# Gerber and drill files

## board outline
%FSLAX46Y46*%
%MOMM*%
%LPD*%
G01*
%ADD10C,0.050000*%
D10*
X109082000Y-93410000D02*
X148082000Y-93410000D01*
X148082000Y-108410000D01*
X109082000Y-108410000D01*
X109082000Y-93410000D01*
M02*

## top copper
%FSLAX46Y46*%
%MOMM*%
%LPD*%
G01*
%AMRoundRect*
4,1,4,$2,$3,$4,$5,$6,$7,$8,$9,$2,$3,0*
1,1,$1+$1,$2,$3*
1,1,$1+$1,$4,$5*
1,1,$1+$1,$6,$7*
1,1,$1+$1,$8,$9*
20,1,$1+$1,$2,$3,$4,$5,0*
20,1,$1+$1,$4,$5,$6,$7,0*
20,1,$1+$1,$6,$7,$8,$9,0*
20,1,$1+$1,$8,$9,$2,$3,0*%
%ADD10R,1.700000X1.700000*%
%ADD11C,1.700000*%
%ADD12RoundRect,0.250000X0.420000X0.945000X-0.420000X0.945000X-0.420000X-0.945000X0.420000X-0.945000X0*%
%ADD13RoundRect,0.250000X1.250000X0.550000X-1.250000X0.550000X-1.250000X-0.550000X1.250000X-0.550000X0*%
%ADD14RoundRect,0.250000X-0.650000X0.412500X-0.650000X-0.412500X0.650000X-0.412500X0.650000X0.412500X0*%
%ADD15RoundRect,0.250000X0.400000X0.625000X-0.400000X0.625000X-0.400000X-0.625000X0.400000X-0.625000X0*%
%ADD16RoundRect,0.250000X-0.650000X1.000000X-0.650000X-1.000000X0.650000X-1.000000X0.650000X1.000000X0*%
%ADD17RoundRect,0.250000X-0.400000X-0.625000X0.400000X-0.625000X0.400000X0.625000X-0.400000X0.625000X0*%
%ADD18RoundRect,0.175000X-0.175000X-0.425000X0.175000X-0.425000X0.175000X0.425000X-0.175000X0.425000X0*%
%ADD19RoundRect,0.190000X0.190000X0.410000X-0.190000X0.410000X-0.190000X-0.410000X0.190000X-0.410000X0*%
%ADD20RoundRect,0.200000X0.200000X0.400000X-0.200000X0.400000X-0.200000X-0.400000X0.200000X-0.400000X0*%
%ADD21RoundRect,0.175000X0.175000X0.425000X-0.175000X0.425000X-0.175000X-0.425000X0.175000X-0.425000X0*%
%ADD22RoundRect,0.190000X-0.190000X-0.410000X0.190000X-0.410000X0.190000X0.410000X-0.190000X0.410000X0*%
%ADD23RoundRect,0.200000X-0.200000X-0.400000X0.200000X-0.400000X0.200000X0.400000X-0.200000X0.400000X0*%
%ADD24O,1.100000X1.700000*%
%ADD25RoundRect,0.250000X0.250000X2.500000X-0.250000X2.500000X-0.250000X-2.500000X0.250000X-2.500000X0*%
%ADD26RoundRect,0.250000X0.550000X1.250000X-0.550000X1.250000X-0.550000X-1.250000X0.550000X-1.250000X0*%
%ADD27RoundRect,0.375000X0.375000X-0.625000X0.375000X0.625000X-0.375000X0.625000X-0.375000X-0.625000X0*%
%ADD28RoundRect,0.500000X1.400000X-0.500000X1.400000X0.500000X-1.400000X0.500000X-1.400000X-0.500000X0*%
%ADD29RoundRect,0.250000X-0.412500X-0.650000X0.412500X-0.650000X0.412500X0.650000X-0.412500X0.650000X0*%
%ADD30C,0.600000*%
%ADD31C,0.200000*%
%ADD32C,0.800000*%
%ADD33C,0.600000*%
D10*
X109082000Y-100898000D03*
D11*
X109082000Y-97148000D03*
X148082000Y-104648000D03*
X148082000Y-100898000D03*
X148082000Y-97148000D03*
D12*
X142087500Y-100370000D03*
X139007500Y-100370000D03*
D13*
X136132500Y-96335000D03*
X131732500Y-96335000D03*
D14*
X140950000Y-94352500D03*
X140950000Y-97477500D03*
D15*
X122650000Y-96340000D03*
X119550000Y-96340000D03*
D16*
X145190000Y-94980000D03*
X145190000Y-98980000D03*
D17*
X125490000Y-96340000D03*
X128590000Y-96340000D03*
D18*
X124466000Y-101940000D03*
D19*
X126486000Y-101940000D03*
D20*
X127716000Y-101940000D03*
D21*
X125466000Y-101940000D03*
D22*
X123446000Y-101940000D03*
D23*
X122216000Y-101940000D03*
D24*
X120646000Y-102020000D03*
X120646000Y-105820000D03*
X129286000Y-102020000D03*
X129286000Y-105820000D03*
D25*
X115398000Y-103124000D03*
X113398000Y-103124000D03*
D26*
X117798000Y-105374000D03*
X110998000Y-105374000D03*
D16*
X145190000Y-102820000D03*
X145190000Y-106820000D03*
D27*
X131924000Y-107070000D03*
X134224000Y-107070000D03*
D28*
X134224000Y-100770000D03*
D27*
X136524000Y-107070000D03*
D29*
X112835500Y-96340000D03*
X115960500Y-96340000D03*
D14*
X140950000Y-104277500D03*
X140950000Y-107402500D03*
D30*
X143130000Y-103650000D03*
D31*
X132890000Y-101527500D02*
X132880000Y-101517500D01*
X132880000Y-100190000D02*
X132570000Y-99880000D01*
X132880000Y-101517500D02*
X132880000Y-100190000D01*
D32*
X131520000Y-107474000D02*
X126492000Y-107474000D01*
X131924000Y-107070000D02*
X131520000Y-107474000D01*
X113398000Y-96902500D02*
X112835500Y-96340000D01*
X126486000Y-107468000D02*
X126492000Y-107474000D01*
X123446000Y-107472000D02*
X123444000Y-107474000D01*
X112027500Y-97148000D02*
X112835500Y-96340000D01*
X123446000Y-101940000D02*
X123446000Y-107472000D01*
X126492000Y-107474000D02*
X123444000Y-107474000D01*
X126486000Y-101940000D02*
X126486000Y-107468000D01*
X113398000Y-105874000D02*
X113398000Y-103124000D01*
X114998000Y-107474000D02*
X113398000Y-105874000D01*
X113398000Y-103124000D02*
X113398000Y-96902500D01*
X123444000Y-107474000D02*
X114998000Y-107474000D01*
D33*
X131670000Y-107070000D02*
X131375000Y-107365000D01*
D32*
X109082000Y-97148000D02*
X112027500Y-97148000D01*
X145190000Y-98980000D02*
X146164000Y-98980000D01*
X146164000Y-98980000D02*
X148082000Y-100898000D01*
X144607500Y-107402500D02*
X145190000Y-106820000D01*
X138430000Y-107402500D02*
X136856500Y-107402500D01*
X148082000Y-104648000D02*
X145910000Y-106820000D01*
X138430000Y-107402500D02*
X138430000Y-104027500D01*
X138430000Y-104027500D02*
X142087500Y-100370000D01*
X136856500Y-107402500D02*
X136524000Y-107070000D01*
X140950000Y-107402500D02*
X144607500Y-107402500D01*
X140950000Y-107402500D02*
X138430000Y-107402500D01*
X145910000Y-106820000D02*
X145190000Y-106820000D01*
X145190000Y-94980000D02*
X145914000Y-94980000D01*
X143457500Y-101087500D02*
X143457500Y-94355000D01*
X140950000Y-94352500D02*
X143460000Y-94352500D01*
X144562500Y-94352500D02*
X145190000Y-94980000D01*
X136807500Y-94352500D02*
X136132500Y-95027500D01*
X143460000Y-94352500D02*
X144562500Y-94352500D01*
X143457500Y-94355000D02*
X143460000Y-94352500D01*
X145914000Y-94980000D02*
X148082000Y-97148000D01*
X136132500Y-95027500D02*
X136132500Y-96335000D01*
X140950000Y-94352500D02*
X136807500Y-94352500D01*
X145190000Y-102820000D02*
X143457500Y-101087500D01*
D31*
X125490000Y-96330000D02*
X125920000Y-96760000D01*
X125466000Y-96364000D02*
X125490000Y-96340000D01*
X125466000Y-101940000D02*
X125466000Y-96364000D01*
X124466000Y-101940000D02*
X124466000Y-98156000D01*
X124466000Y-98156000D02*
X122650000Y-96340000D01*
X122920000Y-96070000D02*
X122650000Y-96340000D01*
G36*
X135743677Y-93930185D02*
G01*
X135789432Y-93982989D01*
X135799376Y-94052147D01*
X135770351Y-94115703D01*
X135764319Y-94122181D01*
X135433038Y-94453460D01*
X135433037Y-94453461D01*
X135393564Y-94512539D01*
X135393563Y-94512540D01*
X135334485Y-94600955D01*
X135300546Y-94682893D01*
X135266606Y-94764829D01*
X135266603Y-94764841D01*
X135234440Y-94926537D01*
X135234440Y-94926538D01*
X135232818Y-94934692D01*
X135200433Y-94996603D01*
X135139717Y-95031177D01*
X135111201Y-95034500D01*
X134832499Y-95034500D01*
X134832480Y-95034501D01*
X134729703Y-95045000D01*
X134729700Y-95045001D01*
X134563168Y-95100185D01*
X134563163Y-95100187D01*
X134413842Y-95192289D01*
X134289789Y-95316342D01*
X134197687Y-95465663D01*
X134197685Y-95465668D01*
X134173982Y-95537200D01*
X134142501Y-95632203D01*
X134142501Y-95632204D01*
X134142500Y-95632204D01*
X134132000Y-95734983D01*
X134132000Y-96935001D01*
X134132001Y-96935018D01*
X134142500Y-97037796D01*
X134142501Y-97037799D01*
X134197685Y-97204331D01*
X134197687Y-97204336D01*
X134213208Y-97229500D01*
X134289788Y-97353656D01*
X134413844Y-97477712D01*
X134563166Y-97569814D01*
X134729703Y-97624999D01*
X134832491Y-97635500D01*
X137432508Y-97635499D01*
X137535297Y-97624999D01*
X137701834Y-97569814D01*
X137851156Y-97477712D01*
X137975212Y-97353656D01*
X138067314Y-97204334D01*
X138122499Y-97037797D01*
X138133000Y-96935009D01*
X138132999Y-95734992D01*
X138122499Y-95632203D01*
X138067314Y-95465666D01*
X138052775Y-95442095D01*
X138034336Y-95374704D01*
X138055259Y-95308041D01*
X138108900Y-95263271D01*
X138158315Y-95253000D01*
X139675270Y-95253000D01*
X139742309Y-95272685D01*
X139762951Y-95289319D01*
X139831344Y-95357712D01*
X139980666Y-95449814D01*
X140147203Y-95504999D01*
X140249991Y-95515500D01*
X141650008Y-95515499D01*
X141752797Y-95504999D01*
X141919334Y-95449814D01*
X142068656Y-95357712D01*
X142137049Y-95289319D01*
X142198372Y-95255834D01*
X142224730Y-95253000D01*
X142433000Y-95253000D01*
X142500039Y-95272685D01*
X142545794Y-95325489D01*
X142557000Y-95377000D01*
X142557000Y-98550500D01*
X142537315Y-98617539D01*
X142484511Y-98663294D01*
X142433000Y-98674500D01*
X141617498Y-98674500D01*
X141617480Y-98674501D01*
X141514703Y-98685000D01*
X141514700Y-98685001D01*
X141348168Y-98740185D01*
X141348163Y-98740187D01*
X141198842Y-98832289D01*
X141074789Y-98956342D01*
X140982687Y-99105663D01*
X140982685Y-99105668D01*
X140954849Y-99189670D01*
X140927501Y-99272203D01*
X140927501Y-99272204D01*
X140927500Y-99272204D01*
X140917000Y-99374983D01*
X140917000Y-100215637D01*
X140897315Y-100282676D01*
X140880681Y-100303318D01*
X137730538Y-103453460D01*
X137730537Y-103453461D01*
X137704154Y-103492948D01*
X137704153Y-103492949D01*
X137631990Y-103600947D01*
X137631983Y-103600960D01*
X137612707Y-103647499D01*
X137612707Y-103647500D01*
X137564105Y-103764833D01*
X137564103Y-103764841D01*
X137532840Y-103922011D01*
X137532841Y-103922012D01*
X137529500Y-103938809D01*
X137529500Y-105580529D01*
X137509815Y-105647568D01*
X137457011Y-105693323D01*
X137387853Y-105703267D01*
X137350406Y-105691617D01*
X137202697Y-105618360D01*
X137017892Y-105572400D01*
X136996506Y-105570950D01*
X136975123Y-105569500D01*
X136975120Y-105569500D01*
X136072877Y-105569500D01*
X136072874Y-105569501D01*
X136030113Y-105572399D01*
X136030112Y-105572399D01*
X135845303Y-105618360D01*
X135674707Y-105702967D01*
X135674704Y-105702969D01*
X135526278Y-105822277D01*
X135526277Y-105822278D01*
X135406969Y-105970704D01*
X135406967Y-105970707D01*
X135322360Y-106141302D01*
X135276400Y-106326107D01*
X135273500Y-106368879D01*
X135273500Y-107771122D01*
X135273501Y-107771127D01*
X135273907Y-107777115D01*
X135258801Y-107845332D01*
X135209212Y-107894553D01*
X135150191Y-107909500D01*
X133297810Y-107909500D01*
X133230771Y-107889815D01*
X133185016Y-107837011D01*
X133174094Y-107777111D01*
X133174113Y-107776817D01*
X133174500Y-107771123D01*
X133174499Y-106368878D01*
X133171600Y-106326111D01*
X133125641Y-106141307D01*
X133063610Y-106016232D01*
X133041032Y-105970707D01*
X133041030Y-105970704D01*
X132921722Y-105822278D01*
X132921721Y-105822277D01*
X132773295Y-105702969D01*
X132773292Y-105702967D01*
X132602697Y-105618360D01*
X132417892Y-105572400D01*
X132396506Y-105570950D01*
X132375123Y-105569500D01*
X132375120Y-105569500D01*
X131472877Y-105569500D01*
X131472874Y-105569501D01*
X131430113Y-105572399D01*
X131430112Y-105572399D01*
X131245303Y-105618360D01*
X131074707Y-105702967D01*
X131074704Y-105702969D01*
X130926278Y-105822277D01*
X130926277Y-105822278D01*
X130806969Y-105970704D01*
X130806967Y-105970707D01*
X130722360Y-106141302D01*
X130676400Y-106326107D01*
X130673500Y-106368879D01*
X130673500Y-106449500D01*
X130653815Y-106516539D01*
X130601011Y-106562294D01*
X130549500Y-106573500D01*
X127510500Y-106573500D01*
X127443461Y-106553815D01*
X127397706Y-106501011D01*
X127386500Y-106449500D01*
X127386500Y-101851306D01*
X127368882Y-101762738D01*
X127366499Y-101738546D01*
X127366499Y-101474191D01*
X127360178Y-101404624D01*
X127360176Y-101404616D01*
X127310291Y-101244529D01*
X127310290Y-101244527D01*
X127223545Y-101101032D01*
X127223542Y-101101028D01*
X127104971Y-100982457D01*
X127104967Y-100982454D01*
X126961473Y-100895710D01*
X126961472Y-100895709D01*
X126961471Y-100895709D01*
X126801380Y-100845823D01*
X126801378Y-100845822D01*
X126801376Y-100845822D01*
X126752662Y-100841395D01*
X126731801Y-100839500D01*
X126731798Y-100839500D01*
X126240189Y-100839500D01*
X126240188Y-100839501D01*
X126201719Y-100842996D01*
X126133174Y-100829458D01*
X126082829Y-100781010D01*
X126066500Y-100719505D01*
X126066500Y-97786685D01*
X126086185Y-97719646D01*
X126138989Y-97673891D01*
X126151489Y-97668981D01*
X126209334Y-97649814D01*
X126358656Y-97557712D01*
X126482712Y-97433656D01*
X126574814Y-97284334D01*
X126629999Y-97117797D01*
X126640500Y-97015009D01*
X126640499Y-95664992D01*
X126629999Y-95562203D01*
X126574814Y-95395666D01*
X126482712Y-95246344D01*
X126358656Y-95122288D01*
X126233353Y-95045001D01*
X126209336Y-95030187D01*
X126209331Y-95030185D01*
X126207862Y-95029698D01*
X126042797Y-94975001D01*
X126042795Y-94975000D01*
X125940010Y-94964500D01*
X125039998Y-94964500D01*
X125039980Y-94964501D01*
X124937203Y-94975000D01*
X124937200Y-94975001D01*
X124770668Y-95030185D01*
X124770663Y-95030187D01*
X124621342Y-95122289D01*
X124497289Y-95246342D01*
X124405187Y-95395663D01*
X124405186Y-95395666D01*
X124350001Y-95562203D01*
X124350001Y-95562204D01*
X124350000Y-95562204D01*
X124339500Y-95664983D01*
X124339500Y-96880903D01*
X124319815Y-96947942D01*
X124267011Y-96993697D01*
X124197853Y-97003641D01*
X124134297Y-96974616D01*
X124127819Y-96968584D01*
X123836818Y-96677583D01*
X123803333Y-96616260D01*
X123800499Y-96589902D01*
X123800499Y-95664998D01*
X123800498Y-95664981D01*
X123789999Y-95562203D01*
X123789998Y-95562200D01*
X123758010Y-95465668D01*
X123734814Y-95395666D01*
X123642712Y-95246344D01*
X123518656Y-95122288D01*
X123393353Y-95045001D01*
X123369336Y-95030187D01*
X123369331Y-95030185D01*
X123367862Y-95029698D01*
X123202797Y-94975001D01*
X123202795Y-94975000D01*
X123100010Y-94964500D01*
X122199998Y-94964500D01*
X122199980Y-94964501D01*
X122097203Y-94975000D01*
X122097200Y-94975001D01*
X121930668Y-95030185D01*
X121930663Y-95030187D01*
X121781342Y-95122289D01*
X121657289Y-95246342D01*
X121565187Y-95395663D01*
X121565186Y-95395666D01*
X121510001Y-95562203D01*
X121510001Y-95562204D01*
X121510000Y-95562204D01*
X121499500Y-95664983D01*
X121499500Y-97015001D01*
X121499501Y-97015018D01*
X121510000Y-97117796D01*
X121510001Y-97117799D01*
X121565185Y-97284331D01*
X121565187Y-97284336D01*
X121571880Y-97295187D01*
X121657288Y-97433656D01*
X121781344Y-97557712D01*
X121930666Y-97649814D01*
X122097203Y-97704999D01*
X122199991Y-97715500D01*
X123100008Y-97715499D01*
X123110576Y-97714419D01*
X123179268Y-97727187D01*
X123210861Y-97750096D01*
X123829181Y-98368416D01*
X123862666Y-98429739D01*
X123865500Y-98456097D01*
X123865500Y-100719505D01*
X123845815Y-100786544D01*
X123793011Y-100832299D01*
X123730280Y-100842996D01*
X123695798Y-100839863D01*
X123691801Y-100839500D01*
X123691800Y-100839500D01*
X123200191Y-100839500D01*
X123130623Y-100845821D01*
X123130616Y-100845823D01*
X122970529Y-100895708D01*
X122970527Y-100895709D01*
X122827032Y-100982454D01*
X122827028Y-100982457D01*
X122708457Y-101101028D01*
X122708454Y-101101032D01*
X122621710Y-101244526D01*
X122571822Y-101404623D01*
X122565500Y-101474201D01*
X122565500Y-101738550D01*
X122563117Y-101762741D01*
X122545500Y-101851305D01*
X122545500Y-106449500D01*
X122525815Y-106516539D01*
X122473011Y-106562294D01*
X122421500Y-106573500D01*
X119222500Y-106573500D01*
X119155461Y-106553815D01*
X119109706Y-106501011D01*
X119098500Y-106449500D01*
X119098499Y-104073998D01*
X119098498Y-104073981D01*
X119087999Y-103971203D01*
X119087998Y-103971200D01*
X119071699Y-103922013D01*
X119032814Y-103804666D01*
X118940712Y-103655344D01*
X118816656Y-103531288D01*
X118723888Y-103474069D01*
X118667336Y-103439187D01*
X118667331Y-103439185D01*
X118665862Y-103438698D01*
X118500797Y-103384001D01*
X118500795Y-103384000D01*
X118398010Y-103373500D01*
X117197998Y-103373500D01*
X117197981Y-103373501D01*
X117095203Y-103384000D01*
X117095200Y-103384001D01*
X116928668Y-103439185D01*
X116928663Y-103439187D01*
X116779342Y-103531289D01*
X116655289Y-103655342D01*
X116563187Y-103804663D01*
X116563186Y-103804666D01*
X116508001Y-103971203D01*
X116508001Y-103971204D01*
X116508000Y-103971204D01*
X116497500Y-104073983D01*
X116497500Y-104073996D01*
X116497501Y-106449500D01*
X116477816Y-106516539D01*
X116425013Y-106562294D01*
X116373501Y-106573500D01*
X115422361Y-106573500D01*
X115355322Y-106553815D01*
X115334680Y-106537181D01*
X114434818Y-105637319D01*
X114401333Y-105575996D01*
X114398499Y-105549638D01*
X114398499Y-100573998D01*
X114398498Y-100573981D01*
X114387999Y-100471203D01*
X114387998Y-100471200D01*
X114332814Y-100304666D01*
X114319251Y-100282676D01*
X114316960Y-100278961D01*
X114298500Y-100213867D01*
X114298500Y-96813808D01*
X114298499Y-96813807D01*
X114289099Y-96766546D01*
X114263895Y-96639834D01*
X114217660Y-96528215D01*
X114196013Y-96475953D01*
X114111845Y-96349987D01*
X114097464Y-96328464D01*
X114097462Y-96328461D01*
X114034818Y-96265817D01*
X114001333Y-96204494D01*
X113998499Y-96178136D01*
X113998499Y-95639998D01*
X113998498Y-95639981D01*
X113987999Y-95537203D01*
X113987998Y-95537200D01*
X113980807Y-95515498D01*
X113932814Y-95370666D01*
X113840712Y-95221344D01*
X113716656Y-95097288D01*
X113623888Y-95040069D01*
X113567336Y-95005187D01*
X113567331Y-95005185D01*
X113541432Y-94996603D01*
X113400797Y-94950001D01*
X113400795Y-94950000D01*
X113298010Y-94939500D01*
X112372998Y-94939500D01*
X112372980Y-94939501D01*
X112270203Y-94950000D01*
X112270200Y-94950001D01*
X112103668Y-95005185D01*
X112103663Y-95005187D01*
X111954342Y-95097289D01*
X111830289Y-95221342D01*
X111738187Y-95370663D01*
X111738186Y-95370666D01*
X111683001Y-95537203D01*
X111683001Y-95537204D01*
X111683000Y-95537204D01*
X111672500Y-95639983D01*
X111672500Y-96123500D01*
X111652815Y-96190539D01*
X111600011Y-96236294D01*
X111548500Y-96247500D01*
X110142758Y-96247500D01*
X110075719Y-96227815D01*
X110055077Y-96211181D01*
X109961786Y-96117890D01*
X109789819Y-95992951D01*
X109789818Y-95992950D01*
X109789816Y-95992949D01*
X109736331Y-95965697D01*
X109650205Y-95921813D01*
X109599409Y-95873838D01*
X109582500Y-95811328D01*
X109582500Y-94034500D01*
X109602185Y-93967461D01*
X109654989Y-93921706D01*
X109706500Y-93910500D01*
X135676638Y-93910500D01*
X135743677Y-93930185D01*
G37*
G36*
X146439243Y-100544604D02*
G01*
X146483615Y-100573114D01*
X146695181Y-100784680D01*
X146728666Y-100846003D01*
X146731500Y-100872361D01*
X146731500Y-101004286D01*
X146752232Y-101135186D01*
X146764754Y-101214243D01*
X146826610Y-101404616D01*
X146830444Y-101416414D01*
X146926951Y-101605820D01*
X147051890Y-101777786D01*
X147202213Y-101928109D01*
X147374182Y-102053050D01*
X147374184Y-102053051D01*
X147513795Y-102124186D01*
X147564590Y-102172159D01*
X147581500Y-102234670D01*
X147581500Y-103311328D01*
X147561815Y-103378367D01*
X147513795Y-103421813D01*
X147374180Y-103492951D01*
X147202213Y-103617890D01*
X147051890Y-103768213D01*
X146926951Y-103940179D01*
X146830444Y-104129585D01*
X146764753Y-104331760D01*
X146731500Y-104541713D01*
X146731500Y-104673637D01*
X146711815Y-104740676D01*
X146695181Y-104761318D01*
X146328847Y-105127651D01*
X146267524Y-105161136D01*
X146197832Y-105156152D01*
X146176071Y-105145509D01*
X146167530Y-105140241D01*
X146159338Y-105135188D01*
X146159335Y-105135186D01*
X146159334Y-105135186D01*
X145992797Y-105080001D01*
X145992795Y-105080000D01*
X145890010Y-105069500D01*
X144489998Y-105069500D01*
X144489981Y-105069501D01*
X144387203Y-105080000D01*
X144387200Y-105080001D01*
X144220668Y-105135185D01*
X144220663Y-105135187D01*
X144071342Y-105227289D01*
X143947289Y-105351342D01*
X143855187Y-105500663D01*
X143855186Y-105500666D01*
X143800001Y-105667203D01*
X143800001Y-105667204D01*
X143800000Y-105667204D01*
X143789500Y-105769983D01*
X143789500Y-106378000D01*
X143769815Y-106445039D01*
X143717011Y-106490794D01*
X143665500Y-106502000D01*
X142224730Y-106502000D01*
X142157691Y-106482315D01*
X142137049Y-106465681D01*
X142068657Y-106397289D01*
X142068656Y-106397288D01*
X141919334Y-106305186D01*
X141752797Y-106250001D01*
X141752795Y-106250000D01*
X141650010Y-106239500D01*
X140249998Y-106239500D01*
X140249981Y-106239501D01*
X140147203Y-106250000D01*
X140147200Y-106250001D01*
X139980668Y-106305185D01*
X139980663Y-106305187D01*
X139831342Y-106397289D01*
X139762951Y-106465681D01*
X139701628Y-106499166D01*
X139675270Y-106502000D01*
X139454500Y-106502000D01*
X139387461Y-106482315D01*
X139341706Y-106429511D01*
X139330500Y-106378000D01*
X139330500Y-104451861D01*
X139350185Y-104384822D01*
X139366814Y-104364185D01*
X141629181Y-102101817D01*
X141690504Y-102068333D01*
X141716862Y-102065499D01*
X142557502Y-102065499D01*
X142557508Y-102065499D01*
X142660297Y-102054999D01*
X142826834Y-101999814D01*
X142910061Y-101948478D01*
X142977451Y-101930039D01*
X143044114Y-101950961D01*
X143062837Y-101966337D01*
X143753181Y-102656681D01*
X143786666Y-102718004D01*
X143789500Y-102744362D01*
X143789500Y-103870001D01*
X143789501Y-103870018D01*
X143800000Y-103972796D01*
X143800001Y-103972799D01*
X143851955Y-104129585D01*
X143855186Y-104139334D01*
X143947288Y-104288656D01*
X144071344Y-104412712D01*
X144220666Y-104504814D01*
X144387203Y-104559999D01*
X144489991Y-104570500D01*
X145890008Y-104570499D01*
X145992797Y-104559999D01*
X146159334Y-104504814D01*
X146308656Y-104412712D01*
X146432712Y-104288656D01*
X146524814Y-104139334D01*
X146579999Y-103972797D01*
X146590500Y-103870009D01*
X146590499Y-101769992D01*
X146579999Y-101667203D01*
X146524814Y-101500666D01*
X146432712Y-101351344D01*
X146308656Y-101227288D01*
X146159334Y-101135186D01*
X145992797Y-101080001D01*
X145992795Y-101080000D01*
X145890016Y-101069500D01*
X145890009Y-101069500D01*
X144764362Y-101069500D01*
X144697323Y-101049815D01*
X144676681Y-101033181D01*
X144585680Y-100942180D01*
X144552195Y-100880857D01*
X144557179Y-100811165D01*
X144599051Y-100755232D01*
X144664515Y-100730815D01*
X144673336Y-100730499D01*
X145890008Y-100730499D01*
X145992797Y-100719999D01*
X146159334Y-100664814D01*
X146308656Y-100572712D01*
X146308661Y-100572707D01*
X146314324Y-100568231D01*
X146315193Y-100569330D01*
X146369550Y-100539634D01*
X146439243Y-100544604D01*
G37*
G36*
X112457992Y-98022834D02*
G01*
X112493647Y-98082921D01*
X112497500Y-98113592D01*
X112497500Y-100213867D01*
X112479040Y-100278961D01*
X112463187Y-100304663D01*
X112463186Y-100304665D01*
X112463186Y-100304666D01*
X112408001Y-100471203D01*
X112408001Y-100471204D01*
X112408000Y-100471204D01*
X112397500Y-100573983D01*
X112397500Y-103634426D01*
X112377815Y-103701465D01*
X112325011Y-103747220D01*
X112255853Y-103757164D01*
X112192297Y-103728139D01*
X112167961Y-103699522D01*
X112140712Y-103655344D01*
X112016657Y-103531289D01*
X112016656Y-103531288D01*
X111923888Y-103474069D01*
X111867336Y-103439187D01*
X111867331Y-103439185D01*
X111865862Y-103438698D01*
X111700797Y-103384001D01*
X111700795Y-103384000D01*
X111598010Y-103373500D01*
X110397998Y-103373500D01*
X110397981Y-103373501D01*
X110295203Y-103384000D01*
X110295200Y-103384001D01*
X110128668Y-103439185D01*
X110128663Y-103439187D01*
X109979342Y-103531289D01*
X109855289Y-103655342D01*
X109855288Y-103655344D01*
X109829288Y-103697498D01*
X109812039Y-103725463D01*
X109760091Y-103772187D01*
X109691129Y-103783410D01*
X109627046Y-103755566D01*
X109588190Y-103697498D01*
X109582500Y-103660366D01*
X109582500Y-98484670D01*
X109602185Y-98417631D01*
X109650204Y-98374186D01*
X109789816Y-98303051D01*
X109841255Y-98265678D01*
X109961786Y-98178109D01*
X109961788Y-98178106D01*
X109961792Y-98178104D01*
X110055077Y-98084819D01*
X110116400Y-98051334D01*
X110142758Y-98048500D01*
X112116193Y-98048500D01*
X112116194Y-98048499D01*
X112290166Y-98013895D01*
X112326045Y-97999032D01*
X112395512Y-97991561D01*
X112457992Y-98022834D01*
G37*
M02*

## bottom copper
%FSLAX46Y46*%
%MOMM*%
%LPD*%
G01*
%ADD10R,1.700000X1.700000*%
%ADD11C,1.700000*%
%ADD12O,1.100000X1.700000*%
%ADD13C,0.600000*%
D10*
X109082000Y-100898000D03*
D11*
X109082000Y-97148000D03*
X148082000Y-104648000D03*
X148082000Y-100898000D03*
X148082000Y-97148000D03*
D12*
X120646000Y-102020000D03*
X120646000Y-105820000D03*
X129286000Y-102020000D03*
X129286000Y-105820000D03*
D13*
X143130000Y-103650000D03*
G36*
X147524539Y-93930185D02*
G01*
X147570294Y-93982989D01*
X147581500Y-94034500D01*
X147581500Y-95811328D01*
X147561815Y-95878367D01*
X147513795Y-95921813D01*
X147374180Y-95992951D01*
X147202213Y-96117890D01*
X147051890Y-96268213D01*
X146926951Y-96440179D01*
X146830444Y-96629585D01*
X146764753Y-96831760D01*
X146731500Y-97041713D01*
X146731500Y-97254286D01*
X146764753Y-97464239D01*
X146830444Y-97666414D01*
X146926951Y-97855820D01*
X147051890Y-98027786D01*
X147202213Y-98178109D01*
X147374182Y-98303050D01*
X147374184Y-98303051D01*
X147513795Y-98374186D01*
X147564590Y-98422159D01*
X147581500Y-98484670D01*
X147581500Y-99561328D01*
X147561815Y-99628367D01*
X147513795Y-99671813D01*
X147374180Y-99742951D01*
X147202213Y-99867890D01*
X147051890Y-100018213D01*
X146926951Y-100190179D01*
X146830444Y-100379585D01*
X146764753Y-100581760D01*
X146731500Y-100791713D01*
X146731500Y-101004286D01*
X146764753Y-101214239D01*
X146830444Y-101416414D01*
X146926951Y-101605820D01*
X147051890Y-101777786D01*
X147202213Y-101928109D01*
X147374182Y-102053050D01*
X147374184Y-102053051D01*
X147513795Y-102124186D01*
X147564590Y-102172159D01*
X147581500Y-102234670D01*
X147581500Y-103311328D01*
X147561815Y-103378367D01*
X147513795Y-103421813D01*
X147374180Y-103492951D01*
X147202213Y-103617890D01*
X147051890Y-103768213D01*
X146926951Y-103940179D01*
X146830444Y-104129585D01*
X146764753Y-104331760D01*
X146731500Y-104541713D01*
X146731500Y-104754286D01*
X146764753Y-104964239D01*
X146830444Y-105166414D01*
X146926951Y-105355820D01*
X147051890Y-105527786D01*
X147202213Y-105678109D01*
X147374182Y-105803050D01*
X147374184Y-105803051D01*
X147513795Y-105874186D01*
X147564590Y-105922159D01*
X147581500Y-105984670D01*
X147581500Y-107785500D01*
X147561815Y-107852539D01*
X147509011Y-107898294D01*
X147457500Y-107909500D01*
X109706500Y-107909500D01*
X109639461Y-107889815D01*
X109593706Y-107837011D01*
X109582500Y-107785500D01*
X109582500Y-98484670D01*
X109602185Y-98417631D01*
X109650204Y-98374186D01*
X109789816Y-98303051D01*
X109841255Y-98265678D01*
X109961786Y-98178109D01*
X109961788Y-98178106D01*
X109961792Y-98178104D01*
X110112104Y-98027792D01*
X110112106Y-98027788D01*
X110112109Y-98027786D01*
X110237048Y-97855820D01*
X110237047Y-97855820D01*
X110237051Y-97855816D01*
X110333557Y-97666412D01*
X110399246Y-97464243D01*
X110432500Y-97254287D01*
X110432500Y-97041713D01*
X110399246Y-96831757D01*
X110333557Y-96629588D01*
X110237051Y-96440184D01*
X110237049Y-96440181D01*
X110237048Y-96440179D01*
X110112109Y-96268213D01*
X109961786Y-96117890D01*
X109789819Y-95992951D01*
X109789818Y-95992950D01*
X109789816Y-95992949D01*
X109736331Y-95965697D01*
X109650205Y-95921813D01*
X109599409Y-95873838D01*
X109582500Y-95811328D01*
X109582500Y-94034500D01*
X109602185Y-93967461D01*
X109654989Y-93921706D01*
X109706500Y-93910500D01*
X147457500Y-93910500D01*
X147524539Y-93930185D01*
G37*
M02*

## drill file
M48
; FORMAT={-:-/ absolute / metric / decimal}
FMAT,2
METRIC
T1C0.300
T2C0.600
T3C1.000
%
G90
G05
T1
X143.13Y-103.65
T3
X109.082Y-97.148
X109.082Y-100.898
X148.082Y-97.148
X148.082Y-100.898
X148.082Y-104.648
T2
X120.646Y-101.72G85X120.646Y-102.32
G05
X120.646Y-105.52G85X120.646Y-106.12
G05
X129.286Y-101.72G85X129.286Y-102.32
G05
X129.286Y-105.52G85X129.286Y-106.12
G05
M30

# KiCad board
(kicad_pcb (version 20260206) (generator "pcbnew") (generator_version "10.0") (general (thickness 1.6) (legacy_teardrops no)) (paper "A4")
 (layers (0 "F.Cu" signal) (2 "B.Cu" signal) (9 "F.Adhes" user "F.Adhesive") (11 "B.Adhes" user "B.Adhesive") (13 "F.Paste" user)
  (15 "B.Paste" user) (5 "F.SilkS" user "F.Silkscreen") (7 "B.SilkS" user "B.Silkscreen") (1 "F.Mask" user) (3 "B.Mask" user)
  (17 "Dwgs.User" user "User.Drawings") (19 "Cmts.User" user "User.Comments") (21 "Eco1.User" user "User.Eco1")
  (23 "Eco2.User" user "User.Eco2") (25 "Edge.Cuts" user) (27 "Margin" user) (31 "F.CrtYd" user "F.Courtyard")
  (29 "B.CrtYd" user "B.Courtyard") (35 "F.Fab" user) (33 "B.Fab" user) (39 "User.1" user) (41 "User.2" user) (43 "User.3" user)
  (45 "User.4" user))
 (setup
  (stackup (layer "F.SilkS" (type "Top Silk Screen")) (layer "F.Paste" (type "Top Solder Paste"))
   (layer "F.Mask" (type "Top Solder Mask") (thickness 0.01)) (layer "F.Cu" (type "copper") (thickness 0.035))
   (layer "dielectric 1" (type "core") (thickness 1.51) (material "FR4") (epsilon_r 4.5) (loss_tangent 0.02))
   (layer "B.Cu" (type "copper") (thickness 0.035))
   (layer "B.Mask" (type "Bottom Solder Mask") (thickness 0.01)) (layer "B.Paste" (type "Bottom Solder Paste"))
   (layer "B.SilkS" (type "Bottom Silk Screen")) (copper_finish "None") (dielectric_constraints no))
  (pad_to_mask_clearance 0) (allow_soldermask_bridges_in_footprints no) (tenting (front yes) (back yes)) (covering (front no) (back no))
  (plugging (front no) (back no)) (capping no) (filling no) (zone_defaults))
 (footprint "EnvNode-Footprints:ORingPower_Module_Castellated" (layer "F.Cu") (at 128.582 100.898)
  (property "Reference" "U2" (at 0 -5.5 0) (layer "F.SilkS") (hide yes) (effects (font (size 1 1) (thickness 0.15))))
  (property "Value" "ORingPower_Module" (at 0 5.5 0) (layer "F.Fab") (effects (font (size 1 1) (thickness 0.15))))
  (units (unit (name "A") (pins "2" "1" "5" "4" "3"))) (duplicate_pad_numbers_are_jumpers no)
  (pad "1" thru_hole rect (at -19.5 0) (size 1.7 1.7) (drill 1) (layers "*.Cu" "*.Mask") (remove_unused_layers no) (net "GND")
   (zone_connect 2))
  (pad "2" thru_hole circle (at -19.5 -3.75) (size 1.7 1.7) (drill 1) (layers "*.Cu" "*.Mask") (remove_unused_layers no) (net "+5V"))
  (pad "3" thru_hole circle (at 19.5 3.75) (size 1.7 1.7) (drill 1) (layers "*.Cu" "*.Mask") (remove_unused_layers no) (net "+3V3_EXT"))
  (pad "4" thru_hole circle (at 19.5 0) (size 1.7 1.7) (drill 1) (layers "*.Cu" "*.Mask") (remove_unused_layers no) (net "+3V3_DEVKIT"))
  (pad "5" thru_hole circle (at 19.5 -3.75) (size 1.7 1.7) (drill 1) (layers "*.Cu" "*.Mask") (remove_unused_layers no) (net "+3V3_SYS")))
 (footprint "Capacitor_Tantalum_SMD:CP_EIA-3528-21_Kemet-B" (layer "F.Cu") (at 140.5475 100.37 180)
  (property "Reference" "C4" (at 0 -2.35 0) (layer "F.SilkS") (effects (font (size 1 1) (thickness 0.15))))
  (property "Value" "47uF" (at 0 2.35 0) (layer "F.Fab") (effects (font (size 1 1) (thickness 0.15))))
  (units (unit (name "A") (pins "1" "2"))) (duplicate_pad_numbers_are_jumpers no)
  (pad "1" smd roundrect (at -1.54 0 180) (size 1.34 2.39) (layers "F.Cu" "F.Mask" "F.Paste") (roundrect_rratio 0.186567) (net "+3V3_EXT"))
  (pad "2" smd roundrect (at 1.54 0 180) (size 1.34 2.39) (layers "F.Cu" "F.Mask" "F.Paste") (roundrect_rratio 0.186567) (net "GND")
   (zone_connect 2)))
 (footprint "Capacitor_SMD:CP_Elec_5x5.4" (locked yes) (layer "F.Cu") (at 133.9325 96.335 180)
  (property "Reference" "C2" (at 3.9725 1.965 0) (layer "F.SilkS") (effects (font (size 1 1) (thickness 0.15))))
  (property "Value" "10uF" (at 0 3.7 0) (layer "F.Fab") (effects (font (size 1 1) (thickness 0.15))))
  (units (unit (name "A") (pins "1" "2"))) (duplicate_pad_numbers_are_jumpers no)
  (pad "1" smd roundrect (at -2.2 0 180) (size 3 1.6) (layers "F.Cu" "F.Mask" "F.Paste") (roundrect_rratio 0.15625) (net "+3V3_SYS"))
  (pad "2" smd roundrect (at 2.2 0 180) (size 3 1.6) (layers "F.Cu" "F.Mask" "F.Paste") (roundrect_rratio 0.15625) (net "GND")
   (zone_connect 2)))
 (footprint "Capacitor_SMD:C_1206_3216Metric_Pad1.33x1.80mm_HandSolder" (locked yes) (layer "F.Cu") (at 140.95 95.915 -90)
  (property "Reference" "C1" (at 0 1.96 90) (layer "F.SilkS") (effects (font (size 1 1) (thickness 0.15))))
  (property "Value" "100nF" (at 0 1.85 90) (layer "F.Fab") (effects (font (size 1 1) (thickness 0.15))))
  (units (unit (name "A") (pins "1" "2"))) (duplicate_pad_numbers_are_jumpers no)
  (pad "1" smd roundrect (at -1.5625 0 270) (size 1.325 1.8) (layers "F.Cu" "F.Mask" "F.Paste") (roundrect_rratio 0.188679) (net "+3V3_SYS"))
  (pad "2" smd roundrect (at 1.5625 0 270) (size 1.325 1.8) (layers "F.Cu" "F.Mask" "F.Paste") (roundrect_rratio 0.188679) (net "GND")
   (zone_connect 2)))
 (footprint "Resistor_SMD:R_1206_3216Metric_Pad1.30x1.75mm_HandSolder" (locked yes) (layer "F.Cu") (at 121.1 96.34 180)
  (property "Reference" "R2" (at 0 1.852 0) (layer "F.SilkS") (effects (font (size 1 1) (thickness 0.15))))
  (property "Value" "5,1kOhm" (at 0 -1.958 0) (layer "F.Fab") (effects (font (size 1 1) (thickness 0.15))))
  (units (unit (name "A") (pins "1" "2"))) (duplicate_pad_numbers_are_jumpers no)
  (pad "1" smd roundrect (at -1.55 0 180) (size 1.3 1.75) (layers "F.Cu" "F.Mask" "F.Paste") (roundrect_rratio 0.192308)
   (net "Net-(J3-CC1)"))
  (pad "2" smd roundrect (at 1.55 0 180) (size 1.3 1.75) (layers "F.Cu" "F.Mask" "F.Paste") (roundrect_rratio 0.192308) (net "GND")
   (zone_connect 2)))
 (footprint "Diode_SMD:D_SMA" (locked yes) (layer "F.Cu") (at 145.19 96.98 -90)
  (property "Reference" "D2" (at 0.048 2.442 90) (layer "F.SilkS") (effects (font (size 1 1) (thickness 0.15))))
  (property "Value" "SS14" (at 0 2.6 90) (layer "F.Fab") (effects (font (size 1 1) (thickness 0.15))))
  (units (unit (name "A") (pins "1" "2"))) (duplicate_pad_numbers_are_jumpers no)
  (pad "1" smd roundrect (at -2 0 270) (size 2.5 1.8) (layers "F.Cu" "F.Mask" "F.Paste") (roundrect_rratio 0.1388888889) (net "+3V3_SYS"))
  (pad "2" smd roundrect (at 2 0 270) (size 2.5 1.8) (layers "F.Cu" "F.Mask" "F.Paste") (roundrect_rratio 0.1388888889) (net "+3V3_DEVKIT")))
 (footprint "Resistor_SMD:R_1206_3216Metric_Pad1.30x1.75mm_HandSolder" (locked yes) (layer "F.Cu") (at 127.04 96.34)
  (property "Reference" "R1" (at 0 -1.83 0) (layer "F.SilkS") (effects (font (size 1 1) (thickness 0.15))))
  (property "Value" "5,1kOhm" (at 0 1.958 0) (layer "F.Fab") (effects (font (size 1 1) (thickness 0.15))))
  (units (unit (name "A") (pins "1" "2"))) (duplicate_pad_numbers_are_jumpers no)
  (pad "1" smd roundrect (at -1.55 0) (size 1.3 1.75) (layers "F.Cu" "F.Mask" "F.Paste") (roundrect_rratio 0.192308) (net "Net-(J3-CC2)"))
  (pad "2" smd roundrect (at 1.55 0) (size 1.3 1.75) (layers "F.Cu" "F.Mask" "F.Paste") (roundrect_rratio 0.192308) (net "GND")
   (zone_connect 2)))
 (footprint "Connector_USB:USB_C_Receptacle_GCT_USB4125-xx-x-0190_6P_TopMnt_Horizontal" (layer "F.Cu") (at 124.966 105.02)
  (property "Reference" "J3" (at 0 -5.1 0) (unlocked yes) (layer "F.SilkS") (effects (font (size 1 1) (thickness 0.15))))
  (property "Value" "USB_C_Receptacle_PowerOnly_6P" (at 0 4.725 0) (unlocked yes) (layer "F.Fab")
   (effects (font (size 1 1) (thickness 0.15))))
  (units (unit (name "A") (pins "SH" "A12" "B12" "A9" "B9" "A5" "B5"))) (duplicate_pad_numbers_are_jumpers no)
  (pad "A5" smd roundrect (at -0.5 -3.08) (size 0.7 1.2) (layers "F.Cu" "F.Mask" "F.Paste") (roundrect_rratio 0.25) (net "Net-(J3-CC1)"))
  (pad "A9" smd roundrect (at 1.52 -3.08 180) (size 0.76 1.2) (layers "F.Cu" "F.Mask" "F.Paste") (roundrect_rratio 0.25) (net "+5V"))
  (pad "A12" smd roundrect (at 2.75 -3.08 180) (size 0.8 1.2) (layers "F.Cu" "F.Mask" "F.Paste") (roundrect_rratio 0.25) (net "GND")
   (zone_connect 2))
  (pad "B5" smd roundrect (at 0.5 -3.08 180) (size 0.7 1.2) (layers "F.Cu" "F.Mask" "F.Paste") (roundrect_rratio 0.25) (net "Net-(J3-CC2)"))
  (pad "B9" smd roundrect (at -1.52 -3.08) (size 0.76 1.2) (layers "F.Cu" "F.Mask" "F.Paste") (roundrect_rratio 0.25) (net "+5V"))
  (pad "B12" smd roundrect (at -2.75 -3.08) (size 0.8 1.2) (layers "F.Cu" "F.Mask" "F.Paste") (roundrect_rratio 0.25) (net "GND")
   (zone_connect 2))
  (pad "SH" thru_hole oval (at -4.32 -3) (size 1.1 1.7) (drill oval 0.6 1.2) (layers "*.Cu" "*.Mask" "F.Paste") (remove_unused_layers no)
   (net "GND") (zone_connect 2))
  (pad "SH" thru_hole oval (at -4.32 0.8) (size 1.1 1.7) (drill oval 0.6 1.2) (layers "*.Cu" "*.Mask" "F.Paste") (remove_unused_layers no)
   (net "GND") (zone_connect 2))
  (pad "SH" thru_hole oval (at 4.32 -3) (size 1.1 1.7) (drill oval 0.6 1.2) (layers "*.Cu" "*.Mask" "F.Paste") (remove_unused_layers no)
   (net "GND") (zone_connect 2))
  (pad "SH" thru_hole oval (at 4.32 0.8) (size 1.1 1.7) (drill oval 0.6 1.2) (layers "*.Cu" "*.Mask" "F.Paste") (remove_unused_layers no)
   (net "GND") (zone_connect 2)))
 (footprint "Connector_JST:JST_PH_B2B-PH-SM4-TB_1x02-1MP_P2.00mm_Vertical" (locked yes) (layer "F.Cu") (at 114.398 103.624 180)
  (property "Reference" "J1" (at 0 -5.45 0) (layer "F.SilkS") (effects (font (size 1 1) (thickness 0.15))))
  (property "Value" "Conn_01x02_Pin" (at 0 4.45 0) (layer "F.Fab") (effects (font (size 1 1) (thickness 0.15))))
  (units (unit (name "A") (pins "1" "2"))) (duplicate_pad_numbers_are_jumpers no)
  (pad "1" smd roundrect (at -1 0.5 180) (size 1 5.5) (layers "F.Cu" "F.Mask" "F.Paste") (roundrect_rratio 0.25) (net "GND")
   (zone_connect 2))
  (pad "2" smd roundrect (at 1 0.5 180) (size 1 5.5) (layers "F.Cu" "F.Mask" "F.Paste") (roundrect_rratio 0.25) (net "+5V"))
  (pad "MP" smd roundrect (at -3.4 -1.75 180) (size 1.6 3) (layers "F.Cu" "F.Mask" "F.Paste") (roundrect_rratio 0.15625))
  (pad "MP" smd roundrect (at 3.4 -1.75 180) (size 1.6 3) (layers "F.Cu" "F.Mask" "F.Paste") (roundrect_rratio 0.15625)))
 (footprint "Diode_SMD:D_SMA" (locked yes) (layer "F.Cu") (at 145.19 104.82 -90)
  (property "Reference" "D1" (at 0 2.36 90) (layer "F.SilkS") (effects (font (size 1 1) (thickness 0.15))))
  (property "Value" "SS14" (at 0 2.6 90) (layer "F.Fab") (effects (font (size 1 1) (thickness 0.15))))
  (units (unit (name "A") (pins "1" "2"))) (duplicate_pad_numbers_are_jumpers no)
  (pad "1" smd roundrect (at -2 0 270) (size 2.5 1.8) (layers "F.Cu" "F.Mask" "F.Paste") (roundrect_rratio 0.1388888889) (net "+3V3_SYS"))
  (pad "2" smd roundrect (at 2 0 270) (size 2.5 1.8) (layers "F.Cu" "F.Mask" "F.Paste") (roundrect_rratio 0.1388888889) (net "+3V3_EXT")))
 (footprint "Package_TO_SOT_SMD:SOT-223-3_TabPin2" (layer "F.Cu") (at 134.224 103.92 90)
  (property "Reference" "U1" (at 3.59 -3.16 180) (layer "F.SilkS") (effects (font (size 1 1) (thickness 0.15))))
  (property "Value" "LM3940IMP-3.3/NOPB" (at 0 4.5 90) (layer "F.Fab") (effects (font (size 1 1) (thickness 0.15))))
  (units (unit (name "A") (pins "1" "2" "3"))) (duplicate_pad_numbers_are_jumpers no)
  (pad "1" smd roundrect (at -3.15 -2.3 90) (size 2 1.5) (layers "F.Cu" "F.Mask" "F.Paste") (roundrect_rratio 0.25) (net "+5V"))
  (pad "2" smd roundrect (at -3.15 0 90) (size 2 1.5) (layers "F.Cu" "F.Mask" "F.Paste") (roundrect_rratio 0.25) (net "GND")
   (zone_connect 2))
  (pad "2" smd roundrect (at 3.15 0 90) (size 2 3.8) (layers "F.Cu" "F.Mask" "F.Paste") (roundrect_rratio 0.25) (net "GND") (zone_connect 2))
  (pad "3" smd roundrect (at -3.15 2.3 90) (size 2 1.5) (layers "F.Cu" "F.Mask" "F.Paste") (roundrect_rratio 0.25) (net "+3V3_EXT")))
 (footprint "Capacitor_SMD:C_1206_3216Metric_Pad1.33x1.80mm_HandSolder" (layer "F.Cu") (at 114.398 96.34)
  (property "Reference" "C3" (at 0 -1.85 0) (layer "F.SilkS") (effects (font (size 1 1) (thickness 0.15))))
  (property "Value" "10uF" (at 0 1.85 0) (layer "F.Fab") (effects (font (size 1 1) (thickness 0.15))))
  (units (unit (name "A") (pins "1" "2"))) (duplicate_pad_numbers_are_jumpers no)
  (pad "1" smd roundrect (at -1.5625 0) (size 1.325 1.8) (layers "F.Cu" "F.Mask" "F.Paste") (roundrect_rratio 0.188679) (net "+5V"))
  (pad "2" smd roundrect (at 1.5625 0) (size 1.325 1.8) (layers "F.Cu" "F.Mask" "F.Paste") (roundrect_rratio 0.188679) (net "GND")
   (zone_connect 2)))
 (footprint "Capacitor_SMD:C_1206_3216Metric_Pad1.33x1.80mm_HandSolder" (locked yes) (layer "F.Cu") (at 140.95 105.84 -90)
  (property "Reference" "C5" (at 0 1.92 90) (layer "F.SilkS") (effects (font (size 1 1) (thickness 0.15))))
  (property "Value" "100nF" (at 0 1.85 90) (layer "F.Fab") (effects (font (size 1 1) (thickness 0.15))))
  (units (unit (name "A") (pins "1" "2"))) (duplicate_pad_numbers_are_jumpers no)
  (pad "1" smd roundrect (at -1.5625 0 270) (size 1.325 1.8) (layers "F.Cu" "F.Mask" "F.Paste") (roundrect_rratio 0.188679) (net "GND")
   (zone_connect 2))
  (pad "2" smd roundrect (at 1.5625 0 270) (size 1.325 1.8) (layers "F.Cu" "F.Mask" "F.Paste") (roundrect_rratio 0.188679) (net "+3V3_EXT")))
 (gr_rect (start 109.082 93.41) (end 148.082 108.41) (stroke (width 0.05) (type solid)) (fill no) (layer "Edge.Cuts"))
 (segment (start 132.89 101.5275) (end 132.88 101.5175) (width 0.2) (layer "F.Cu") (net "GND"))
 (segment (start 132.88 100.19) (end 132.57 99.88) (width 0.2) (layer "F.Cu") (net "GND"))
 (segment (start 132.88 101.5175) (end 132.88 100.19) (width 0.2) (layer "F.Cu") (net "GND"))
 (via (at 143.13 103.65) (size 0.6) (drill 0.3) (layers "F.Cu" "B.Cu") (free yes) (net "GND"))
 (segment (start 131.52 107.474) (end 126.492 107.474) (width 0.8) (layer "F.Cu") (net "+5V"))
 (segment (start 131.924 107.07) (end 131.52 107.474) (width 0.8) (layer "F.Cu") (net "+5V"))
 (segment (start 113.398 96.9025) (end 112.8355 96.34) (width 0.8) (layer "F.Cu") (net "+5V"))
 (segment (start 126.486 107.468) (end 126.492 107.474) (width 0.8) (layer "F.Cu") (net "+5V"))
 (segment (start 123.446 107.472) (end 123.444 107.474) (width 0.8) (layer "F.Cu") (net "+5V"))
 (segment (start 112.0275 97.148) (end 112.8355 96.34) (width 0.8) (layer "F.Cu") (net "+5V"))
 (segment (start 123.446 101.94) (end 123.446 107.472) (width 0.8) (layer "F.Cu") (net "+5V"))
 (segment (start 126.492 107.474) (end 123.444 107.474) (width 0.8) (layer "F.Cu") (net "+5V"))
 (segment (start 126.486 101.94) (end 126.486 107.468) (width 0.8) (layer "F.Cu") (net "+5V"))
 (segment (start 113.398 105.874) (end 113.398 103.124) (width 0.8) (layer "F.Cu") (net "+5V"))
 (segment (start 114.998 107.474) (end 113.398 105.874) (width 0.8) (layer "F.Cu") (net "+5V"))
 (segment (start 113.398 103.124) (end 113.398 96.9025) (width 0.8) (layer "F.Cu") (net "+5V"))
 (segment (start 123.444 107.474) (end 114.998 107.474) (width 0.8) (layer "F.Cu") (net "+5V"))
 (segment (start 131.67 107.07) (end 131.375 107.365) (width 0.6) (layer "F.Cu") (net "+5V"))
 (segment (start 109.082 97.148) (end 112.0275 97.148) (width 0.8) (layer "F.Cu") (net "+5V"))
 (segment (start 145.19 98.98) (end 146.164 98.98) (width 0.8) (layer "F.Cu") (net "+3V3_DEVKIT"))
 (segment (start 146.164 98.98) (end 148.082 100.898) (width 0.8) (layer "F.Cu") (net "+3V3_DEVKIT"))
 (segment (start 144.6075 107.4025) (end 145.19 106.82) (width 0.8) (layer "F.Cu") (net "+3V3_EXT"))
 (segment (start 138.43 107.4025) (end 136.8565 107.4025) (width 0.8) (layer "F.Cu") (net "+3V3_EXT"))
 (segment (start 148.082 104.648) (end 145.91 106.82) (width 0.8) (layer "F.Cu") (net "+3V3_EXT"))
 (segment (start 138.43 107.4025) (end 138.43 104.0275) (width 0.8) (layer "F.Cu") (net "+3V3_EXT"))
 (segment (start 138.43 104.0275) (end 142.0875 100.37) (width 0.8) (layer "F.Cu") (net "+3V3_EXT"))
 (segment (start 136.8565 107.4025) (end 136.524 107.07) (width 0.8) (layer "F.Cu") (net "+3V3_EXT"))
 (segment (start 140.95 107.4025) (end 144.6075 107.4025) (width 0.8) (layer "F.Cu") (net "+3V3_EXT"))
 (segment (start 140.95 107.4025) (end 138.43 107.4025) (width 0.8) (layer "F.Cu") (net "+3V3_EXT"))
 (segment (start 145.91 106.82) (end 145.19 106.82) (width 0.8) (layer "F.Cu") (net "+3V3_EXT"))
 (segment (start 145.19 94.98) (end 145.914 94.98) (width 0.8) (layer "F.Cu") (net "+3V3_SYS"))
 (segment (start 143.4575 101.0875) (end 143.4575 94.355) (width 0.8) (layer "F.Cu") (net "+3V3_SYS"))
 (segment (start 140.95 94.3525) (end 143.46 94.3525) (width 0.8) (layer "F.Cu") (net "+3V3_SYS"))
 (segment (start 144.5625 94.3525) (end 145.19 94.98) (width 0.8) (layer "F.Cu") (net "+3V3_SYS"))
 (segment (start 136.8075 94.3525) (end 136.1325 95.0275) (width 0.8) (layer "F.Cu") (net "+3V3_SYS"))
 (segment (start 143.46 94.3525) (end 144.5625 94.3525) (width 0.8) (layer "F.Cu") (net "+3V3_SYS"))
 (segment (start 143.4575 94.355) (end 143.46 94.3525) (width 0.8) (layer "F.Cu") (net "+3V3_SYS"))
 (segment (start 145.914 94.98) (end 148.082 97.148) (width 0.8) (layer "F.Cu") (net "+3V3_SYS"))
 (segment (start 136.1325 95.0275) (end 136.1325 96.335) (width 0.8) (layer "F.Cu") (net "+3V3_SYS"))
 (segment (start 140.95 94.3525) (end 136.8075 94.3525) (width 0.8) (layer "F.Cu") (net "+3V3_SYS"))
 (segment (start 145.19 102.82) (end 143.4575 101.0875) (width 0.8) (layer "F.Cu") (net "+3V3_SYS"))
 (segment (start 125.49 96.33) (end 125.92 96.76) (width 0.2) (layer "F.Cu") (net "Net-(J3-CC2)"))
 (segment (start 125.466 96.364) (end 125.49 96.34) (width 0.2) (layer "F.Cu") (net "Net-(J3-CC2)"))
 (segment (start 125.466 101.94) (end 125.466 96.364) (width 0.2) (layer "F.Cu") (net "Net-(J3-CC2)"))
 (segment (start 124.466 101.94) (end 124.466 98.156) (width 0.2) (layer "F.Cu") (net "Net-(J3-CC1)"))
 (segment (start 124.466 98.156) (end 122.65 96.34) (width 0.2) (layer "F.Cu") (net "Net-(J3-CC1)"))
 (segment (start 122.92 96.07) (end 122.65 96.34) (width 0.2) (layer "F.Cu") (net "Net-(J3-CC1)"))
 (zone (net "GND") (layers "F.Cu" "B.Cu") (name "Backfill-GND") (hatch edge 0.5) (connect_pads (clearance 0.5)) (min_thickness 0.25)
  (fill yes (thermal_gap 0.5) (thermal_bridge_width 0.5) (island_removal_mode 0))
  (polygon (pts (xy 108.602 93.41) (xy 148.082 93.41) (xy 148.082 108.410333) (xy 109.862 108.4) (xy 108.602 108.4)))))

